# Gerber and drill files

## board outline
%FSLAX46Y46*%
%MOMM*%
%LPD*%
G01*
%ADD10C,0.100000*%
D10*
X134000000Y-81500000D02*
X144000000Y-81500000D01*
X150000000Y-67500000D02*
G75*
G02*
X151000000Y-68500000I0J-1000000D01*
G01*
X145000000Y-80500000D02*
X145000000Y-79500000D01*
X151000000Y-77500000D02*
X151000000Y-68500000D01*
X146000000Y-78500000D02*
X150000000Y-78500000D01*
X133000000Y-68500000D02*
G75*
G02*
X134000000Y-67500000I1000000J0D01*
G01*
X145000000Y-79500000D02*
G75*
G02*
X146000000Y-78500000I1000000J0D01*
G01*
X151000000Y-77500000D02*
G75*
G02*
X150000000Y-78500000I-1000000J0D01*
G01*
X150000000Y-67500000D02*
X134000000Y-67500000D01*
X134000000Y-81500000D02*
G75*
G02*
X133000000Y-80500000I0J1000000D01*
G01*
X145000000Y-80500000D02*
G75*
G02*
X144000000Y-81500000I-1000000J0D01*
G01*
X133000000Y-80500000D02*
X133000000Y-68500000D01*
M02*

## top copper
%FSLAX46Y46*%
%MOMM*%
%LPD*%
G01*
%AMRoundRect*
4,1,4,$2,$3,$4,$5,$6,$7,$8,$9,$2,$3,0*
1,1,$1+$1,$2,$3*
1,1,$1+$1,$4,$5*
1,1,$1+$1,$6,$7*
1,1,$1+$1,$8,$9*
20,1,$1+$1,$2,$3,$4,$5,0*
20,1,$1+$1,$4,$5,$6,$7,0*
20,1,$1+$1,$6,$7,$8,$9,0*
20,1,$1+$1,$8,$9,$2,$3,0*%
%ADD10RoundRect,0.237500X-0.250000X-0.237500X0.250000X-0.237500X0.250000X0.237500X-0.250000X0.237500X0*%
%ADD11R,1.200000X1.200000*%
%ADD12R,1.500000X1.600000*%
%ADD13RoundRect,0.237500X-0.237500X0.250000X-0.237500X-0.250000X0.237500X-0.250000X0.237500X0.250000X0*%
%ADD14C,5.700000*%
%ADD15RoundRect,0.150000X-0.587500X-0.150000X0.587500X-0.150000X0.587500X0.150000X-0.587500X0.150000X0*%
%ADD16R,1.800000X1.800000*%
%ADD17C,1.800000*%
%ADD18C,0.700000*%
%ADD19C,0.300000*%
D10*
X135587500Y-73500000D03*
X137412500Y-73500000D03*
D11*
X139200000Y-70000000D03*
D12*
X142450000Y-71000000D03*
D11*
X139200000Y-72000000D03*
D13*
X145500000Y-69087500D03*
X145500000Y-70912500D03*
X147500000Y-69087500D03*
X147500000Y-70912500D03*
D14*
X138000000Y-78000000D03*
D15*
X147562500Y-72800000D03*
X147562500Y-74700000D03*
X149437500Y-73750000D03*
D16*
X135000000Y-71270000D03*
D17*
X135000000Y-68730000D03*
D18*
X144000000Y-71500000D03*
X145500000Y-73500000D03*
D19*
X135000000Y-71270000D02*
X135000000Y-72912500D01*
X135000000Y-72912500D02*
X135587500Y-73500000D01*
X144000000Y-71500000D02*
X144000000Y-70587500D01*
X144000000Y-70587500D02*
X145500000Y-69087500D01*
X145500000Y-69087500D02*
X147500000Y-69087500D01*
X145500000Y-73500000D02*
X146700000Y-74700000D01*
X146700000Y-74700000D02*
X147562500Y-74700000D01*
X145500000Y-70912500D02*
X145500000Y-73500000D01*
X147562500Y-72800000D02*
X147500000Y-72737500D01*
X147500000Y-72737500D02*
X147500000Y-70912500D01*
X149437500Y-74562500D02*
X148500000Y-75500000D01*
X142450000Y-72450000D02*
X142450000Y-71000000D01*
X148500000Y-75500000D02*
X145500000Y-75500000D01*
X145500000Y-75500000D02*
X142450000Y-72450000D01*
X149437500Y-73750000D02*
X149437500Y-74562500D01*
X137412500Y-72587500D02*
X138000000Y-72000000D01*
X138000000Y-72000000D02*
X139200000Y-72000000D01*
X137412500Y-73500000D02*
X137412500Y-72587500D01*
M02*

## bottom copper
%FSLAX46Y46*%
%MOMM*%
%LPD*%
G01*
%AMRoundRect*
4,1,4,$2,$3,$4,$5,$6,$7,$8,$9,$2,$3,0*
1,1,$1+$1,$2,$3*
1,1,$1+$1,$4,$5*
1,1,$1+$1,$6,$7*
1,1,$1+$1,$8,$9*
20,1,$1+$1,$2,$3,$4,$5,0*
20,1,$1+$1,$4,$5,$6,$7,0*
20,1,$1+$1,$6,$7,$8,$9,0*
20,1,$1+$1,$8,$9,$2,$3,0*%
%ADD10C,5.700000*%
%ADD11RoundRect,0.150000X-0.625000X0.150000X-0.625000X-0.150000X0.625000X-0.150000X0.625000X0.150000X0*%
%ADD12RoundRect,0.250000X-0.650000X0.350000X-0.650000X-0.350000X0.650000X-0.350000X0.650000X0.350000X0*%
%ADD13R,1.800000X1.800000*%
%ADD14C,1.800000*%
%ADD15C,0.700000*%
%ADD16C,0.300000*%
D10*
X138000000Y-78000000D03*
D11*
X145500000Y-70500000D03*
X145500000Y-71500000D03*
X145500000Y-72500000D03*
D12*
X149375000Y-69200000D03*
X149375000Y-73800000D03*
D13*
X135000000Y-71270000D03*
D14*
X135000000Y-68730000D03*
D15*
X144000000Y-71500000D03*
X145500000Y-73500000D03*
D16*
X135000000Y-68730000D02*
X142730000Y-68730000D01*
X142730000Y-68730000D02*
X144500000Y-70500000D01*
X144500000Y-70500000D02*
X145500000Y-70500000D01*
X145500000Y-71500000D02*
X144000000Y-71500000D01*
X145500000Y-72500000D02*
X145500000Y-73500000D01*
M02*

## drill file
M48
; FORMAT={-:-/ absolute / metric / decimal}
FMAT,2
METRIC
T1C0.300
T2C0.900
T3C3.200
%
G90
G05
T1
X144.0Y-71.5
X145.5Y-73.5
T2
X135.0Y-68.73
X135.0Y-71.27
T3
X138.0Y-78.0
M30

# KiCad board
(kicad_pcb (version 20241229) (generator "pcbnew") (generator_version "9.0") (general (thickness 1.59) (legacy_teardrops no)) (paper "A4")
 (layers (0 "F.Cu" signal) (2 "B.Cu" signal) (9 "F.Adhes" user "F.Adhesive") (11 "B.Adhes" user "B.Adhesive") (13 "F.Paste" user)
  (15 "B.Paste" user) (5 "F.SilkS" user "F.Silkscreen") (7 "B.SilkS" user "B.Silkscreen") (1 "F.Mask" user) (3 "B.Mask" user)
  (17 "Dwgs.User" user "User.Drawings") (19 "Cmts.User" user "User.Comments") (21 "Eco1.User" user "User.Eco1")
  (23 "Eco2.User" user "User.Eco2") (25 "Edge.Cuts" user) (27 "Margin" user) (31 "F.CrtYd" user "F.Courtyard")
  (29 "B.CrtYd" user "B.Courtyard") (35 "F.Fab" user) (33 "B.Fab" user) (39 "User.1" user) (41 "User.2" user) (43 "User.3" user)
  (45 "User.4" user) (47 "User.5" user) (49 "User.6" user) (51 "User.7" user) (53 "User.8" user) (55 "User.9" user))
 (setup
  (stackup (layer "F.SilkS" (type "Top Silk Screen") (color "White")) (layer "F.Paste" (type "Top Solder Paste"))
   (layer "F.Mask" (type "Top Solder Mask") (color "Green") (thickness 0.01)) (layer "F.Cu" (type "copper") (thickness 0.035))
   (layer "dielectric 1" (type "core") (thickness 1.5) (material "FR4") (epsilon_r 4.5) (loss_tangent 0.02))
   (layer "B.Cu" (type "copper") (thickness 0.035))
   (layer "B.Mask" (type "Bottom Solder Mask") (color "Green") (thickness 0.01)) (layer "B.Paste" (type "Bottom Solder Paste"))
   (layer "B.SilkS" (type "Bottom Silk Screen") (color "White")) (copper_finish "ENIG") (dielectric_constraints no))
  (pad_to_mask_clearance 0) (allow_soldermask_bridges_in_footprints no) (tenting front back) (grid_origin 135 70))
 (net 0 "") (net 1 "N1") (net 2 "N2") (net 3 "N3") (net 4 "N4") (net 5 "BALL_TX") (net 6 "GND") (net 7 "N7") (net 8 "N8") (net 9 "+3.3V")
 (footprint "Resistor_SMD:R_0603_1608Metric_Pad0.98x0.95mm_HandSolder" (layer "F.Cu") (at 136.5 73.5)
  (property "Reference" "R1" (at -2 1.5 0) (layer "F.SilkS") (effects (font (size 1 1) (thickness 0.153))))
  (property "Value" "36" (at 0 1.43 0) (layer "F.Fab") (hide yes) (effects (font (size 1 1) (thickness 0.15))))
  (pad "1" smd roundrect (at -0.9125 0) (size 0.975 0.95) (layers "F.Cu" "F.Mask" "F.Paste") (roundrect_rratio 0.25) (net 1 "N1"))
  (pad "2" smd roundrect (at 0.9125 0) (size 0.975 0.95) (layers "F.Cu" "F.Mask" "F.Paste") (roundrect_rratio 0.25) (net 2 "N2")))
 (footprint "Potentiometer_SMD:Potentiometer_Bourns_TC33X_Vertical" (layer "F.Cu") (at 141 71)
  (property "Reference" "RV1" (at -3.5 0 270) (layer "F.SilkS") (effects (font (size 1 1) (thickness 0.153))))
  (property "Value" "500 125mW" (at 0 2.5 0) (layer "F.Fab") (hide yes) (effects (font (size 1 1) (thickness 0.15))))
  (pad "1" smd rect (at -1.8 -1) (size 1.2 1.2) (layers "F.Cu" "F.Mask" "F.Paste") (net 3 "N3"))
  (pad "2" smd rect (at 1.45 0) (size 1.5 1.6) (layers "F.Cu" "F.Mask" "F.Paste") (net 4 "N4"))
  (pad "3" smd rect (at -1.8 1) (size 1.2 1.2) (layers "F.Cu" "F.Mask" "F.Paste") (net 2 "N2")))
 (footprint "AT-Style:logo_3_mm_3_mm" (layer "F.Cu") (at 142 74.5)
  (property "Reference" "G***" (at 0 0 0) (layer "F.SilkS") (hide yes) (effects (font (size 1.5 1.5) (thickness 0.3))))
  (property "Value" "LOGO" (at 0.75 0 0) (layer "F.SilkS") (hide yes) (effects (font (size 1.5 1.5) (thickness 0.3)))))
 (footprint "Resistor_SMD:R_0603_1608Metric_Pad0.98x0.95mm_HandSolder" (layer "F.Cu") (at 145.5 70 -90)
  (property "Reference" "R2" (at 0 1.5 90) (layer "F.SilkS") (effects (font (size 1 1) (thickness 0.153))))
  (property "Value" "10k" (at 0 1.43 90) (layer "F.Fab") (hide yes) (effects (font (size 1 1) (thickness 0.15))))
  (pad "1" smd roundrect (at -0.9125 0 270) (size 0.975 0.95) (layers "F.Cu" "F.Mask" "F.Paste") (roundrect_rratio 0.25) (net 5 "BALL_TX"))
  (pad "2" smd roundrect (at 0.9125 0 270) (size 0.975 0.95) (layers "F.Cu" "F.Mask" "F.Paste") (roundrect_rratio 0.25) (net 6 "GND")))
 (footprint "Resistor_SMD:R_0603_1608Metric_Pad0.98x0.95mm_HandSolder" (layer "F.Cu") (at 147.5 70 -90)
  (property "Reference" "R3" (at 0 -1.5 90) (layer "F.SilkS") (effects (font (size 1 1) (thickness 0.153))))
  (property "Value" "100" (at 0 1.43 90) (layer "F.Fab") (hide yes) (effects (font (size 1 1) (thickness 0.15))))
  (pad "1" smd roundrect (at -0.9125 0 270) (size 0.975 0.95) (layers "F.Cu" "F.Mask" "F.Paste") (roundrect_rratio 0.25) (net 5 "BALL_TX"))
  (pad "2" smd roundrect (at 0.9125 0 270) (size 0.975 0.95) (layers "F.Cu" "F.Mask" "F.Paste") (roundrect_rratio 0.25) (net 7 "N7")))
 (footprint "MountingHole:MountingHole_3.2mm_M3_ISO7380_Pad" (layer "F.Cu") (at 138 78)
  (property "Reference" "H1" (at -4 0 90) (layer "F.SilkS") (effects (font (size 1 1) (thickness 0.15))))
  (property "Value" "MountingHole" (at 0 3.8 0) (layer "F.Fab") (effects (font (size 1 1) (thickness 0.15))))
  (pad "1" thru_hole circle (at 0 0) (size 5.7 5.7) (drill 3.2) (layers "*.Cu" "*.Mask") (remove_unused_layers no) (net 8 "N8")
   (zone_connect 2)))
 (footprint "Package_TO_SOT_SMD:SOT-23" (layer "F.Cu") (at 148.5 73.75)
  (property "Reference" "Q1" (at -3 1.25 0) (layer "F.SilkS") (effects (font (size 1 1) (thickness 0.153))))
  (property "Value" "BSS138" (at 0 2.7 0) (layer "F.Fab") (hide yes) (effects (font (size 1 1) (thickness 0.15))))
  (pad "1" smd roundrect (at -0.9375 -0.95) (size 1.475 0.6) (layers "F.Cu" "F.Mask" "F.Paste") (roundrect_rratio 0.25) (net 7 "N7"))
  (pad "2" smd roundrect (at -0.9375 0.95) (size 1.475 0.6) (layers "F.Cu" "F.Mask" "F.Paste") (roundrect_rratio 0.25) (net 6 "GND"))
  (pad "3" smd roundrect (at 0.9375 0) (size 1.475 0.6) (layers "F.Cu" "F.Mask" "F.Paste") (roundrect_rratio 0.25) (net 4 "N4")))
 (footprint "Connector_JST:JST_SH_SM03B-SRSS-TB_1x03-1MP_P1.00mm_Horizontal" (layer "B.Cu") (at 147.5 71.5 -90)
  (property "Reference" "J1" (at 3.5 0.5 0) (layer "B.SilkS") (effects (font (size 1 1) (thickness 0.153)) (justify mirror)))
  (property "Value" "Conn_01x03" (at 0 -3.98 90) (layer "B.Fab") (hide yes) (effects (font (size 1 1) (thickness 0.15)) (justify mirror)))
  (pad "1" smd roundrect (at -1 2 270) (size 0.6 1.55) (layers "B.Cu" "B.Mask" "B.Paste") (roundrect_rratio 0.25) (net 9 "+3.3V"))
  (pad "2" smd roundrect (at 0 2 270) (size 0.6 1.55) (layers "B.Cu" "B.Mask" "B.Paste") (roundrect_rratio 0.25) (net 5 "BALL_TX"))
  (pad "3" smd roundrect (at 1 2 270) (size 0.6 1.55) (layers "B.Cu" "B.Mask" "B.Paste") (roundrect_rratio 0.25) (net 6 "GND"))
  (pad "MP" smd roundrect (at -2.3 -1.875 270) (size 1.2 1.8) (layers "B.Cu" "B.Mask" "B.Paste") (roundrect_rratio 0.208333))
  (pad "MP" smd roundrect (at 2.3 -1.875 270) (size 1.2 1.8) (layers "B.Cu" "B.Mask" "B.Paste") (roundrect_rratio 0.208333)))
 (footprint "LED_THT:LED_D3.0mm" (layer "B.Cu") (at 135 71.27 90)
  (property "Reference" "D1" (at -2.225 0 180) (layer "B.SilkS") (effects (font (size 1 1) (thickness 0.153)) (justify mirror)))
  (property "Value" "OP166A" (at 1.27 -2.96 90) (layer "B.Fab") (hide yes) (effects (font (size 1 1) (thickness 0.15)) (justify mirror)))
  (pad "1" thru_hole rect (at 0 0 90) (size 1.8 1.8) (drill 0.9) (layers "*.Cu" "*.Mask") (remove_unused_layers no) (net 1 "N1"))
  (pad "2" thru_hole circle (at 2.54 0 90) (size 1.8 1.8) (drill 0.9) (layers "*.Cu" "*.Mask") (remove_unused_layers no) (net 9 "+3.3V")))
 (gr_line (start 134 81.5) (end 144 81.5) (stroke (width 0.1) (type default)) (layer "Edge.Cuts"))
 (gr_arc (start 150 67.5) (mid 150.707107 67.792893) (end 151 68.5) (stroke (width 0.1) (type default)) (layer "Edge.Cuts"))
 (gr_line (start 145 80.5) (end 145 79.5) (stroke (width 0.1) (type default)) (layer "Edge.Cuts"))
 (gr_line (start 151 77.5) (end 151 68.5) (stroke (width 0.1) (type default)) (layer "Edge.Cuts"))
 (gr_line (start 146 78.5) (end 150 78.5) (stroke (width 0.1) (type default)) (layer "Edge.Cuts"))
 (gr_arc (start 133 68.5) (mid 133.292893 67.792893) (end 134 67.5) (stroke (width 0.1) (type default)) (layer "Edge.Cuts"))
 (gr_arc (start 145 79.5) (mid 145.292893 78.792893) (end 146 78.5) (stroke (width 0.1) (type default)) (layer "Edge.Cuts"))
 (gr_arc (start 151 77.5) (mid 150.707107 78.207107) (end 150 78.5) (stroke (width 0.1) (type default)) (layer "Edge.Cuts"))
 (gr_line (start 150 67.5) (end 134 67.5) (stroke (width 0.1) (type default)) (layer "Edge.Cuts"))
 (gr_arc (start 134 81.5) (mid 133.292893 81.207107) (end 133 80.5) (stroke (width 0.1) (type default)) (layer "Edge.Cuts"))
 (gr_arc (start 145 80.5) (mid 144.707107 81.207107) (end 144 81.5) (stroke (width 0.1) (type default)) (layer "Edge.Cuts"))
 (gr_line (start 133 80.5) (end 133 68.5) (stroke (width 0.1) (type default)) (layer "Edge.Cuts"))
 (segment (start 135 71.27) (end 135 72.9125) (width 0.3) (layer "F.Cu") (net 1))
 (segment (start 135 72.9125) (end 135.5875 73.5) (width 0.3) (layer "F.Cu") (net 1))
 (segment (start 135 68.73) (end 142.73 68.73) (width 0.3) (layer "B.Cu") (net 9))
 (segment (start 142.73 68.73) (end 144.5 70.5) (width 0.3) (layer "B.Cu") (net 9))
 (segment (start 144.5 70.5) (end 145.5 70.5) (width 0.3) (layer "B.Cu") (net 9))
 (segment (start 144 71.5) (end 144 70.5875) (width 0.3) (layer "F.Cu") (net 5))
 (segment (start 144 70.5875) (end 145.5 69.0875) (width 0.3) (layer "F.Cu") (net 5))
 (segment (start 145.5 69.0875) (end 147.5 69.0875) (width 0.3) (layer "F.Cu") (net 5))
 (via (at 144 71.5) (size 0.7) (drill 0.3) (layers "F.Cu" "B.Cu") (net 5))
 (segment (start 145.5 71.5) (end 144 71.5) (width 0.3) (layer "B.Cu") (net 5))
 (segment (start 145.5 73.5) (end 146.7 74.7) (width 0.3) (layer "F.Cu") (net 6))
 (segment (start 146.7 74.7) (end 147.5625 74.7) (width 0.3) (layer "F.Cu") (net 6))
 (segment (start 145.5 70.9125) (end 145.5 73.5) (width 0.3) (layer "F.Cu") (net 6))
 (via (at 145.5 73.5) (size 0.7) (drill 0.3) (layers "F.Cu" "B.Cu") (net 6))
 (segment (start 145.5 72.5) (end 145.5 73.5) (width 0.3) (layer "B.Cu") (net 6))
 (segment (start 147.5625 72.8) (end 147.5 72.7375) (width 0.3) (layer "F.Cu") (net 7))
 (segment (start 147.5 72.7375) (end 147.5 70.9125) (width 0.3) (layer "F.Cu") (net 7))
 (segment (start 149.4375 74.5625) (end 148.5 75.5) (width 0.3) (layer "F.Cu") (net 4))
 (segment (start 142.45 72.45) (end 142.45 71) (width 0.3) (layer "F.Cu") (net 4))
 (segment (start 148.5 75.5) (end 145.5 75.5) (width 0.3) (layer "F.Cu") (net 4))
 (segment (start 145.5 75.5) (end 142.45 72.45) (width 0.3) (layer "F.Cu") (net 4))
 (segment (start 149.4375 73.75) (end 149.4375 74.5625) (width 0.3) (layer "F.Cu") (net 4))
 (segment (start 137.4125 72.5875) (end 138 72) (width 0.3) (layer "F.Cu") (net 2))
 (segment (start 138 72) (end 139.2 72) (width 0.3) (layer "F.Cu") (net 2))
 (segment (start 137.4125 73.5) (end 137.4125 72.5875) (width 0.3) (layer "F.Cu") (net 2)))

